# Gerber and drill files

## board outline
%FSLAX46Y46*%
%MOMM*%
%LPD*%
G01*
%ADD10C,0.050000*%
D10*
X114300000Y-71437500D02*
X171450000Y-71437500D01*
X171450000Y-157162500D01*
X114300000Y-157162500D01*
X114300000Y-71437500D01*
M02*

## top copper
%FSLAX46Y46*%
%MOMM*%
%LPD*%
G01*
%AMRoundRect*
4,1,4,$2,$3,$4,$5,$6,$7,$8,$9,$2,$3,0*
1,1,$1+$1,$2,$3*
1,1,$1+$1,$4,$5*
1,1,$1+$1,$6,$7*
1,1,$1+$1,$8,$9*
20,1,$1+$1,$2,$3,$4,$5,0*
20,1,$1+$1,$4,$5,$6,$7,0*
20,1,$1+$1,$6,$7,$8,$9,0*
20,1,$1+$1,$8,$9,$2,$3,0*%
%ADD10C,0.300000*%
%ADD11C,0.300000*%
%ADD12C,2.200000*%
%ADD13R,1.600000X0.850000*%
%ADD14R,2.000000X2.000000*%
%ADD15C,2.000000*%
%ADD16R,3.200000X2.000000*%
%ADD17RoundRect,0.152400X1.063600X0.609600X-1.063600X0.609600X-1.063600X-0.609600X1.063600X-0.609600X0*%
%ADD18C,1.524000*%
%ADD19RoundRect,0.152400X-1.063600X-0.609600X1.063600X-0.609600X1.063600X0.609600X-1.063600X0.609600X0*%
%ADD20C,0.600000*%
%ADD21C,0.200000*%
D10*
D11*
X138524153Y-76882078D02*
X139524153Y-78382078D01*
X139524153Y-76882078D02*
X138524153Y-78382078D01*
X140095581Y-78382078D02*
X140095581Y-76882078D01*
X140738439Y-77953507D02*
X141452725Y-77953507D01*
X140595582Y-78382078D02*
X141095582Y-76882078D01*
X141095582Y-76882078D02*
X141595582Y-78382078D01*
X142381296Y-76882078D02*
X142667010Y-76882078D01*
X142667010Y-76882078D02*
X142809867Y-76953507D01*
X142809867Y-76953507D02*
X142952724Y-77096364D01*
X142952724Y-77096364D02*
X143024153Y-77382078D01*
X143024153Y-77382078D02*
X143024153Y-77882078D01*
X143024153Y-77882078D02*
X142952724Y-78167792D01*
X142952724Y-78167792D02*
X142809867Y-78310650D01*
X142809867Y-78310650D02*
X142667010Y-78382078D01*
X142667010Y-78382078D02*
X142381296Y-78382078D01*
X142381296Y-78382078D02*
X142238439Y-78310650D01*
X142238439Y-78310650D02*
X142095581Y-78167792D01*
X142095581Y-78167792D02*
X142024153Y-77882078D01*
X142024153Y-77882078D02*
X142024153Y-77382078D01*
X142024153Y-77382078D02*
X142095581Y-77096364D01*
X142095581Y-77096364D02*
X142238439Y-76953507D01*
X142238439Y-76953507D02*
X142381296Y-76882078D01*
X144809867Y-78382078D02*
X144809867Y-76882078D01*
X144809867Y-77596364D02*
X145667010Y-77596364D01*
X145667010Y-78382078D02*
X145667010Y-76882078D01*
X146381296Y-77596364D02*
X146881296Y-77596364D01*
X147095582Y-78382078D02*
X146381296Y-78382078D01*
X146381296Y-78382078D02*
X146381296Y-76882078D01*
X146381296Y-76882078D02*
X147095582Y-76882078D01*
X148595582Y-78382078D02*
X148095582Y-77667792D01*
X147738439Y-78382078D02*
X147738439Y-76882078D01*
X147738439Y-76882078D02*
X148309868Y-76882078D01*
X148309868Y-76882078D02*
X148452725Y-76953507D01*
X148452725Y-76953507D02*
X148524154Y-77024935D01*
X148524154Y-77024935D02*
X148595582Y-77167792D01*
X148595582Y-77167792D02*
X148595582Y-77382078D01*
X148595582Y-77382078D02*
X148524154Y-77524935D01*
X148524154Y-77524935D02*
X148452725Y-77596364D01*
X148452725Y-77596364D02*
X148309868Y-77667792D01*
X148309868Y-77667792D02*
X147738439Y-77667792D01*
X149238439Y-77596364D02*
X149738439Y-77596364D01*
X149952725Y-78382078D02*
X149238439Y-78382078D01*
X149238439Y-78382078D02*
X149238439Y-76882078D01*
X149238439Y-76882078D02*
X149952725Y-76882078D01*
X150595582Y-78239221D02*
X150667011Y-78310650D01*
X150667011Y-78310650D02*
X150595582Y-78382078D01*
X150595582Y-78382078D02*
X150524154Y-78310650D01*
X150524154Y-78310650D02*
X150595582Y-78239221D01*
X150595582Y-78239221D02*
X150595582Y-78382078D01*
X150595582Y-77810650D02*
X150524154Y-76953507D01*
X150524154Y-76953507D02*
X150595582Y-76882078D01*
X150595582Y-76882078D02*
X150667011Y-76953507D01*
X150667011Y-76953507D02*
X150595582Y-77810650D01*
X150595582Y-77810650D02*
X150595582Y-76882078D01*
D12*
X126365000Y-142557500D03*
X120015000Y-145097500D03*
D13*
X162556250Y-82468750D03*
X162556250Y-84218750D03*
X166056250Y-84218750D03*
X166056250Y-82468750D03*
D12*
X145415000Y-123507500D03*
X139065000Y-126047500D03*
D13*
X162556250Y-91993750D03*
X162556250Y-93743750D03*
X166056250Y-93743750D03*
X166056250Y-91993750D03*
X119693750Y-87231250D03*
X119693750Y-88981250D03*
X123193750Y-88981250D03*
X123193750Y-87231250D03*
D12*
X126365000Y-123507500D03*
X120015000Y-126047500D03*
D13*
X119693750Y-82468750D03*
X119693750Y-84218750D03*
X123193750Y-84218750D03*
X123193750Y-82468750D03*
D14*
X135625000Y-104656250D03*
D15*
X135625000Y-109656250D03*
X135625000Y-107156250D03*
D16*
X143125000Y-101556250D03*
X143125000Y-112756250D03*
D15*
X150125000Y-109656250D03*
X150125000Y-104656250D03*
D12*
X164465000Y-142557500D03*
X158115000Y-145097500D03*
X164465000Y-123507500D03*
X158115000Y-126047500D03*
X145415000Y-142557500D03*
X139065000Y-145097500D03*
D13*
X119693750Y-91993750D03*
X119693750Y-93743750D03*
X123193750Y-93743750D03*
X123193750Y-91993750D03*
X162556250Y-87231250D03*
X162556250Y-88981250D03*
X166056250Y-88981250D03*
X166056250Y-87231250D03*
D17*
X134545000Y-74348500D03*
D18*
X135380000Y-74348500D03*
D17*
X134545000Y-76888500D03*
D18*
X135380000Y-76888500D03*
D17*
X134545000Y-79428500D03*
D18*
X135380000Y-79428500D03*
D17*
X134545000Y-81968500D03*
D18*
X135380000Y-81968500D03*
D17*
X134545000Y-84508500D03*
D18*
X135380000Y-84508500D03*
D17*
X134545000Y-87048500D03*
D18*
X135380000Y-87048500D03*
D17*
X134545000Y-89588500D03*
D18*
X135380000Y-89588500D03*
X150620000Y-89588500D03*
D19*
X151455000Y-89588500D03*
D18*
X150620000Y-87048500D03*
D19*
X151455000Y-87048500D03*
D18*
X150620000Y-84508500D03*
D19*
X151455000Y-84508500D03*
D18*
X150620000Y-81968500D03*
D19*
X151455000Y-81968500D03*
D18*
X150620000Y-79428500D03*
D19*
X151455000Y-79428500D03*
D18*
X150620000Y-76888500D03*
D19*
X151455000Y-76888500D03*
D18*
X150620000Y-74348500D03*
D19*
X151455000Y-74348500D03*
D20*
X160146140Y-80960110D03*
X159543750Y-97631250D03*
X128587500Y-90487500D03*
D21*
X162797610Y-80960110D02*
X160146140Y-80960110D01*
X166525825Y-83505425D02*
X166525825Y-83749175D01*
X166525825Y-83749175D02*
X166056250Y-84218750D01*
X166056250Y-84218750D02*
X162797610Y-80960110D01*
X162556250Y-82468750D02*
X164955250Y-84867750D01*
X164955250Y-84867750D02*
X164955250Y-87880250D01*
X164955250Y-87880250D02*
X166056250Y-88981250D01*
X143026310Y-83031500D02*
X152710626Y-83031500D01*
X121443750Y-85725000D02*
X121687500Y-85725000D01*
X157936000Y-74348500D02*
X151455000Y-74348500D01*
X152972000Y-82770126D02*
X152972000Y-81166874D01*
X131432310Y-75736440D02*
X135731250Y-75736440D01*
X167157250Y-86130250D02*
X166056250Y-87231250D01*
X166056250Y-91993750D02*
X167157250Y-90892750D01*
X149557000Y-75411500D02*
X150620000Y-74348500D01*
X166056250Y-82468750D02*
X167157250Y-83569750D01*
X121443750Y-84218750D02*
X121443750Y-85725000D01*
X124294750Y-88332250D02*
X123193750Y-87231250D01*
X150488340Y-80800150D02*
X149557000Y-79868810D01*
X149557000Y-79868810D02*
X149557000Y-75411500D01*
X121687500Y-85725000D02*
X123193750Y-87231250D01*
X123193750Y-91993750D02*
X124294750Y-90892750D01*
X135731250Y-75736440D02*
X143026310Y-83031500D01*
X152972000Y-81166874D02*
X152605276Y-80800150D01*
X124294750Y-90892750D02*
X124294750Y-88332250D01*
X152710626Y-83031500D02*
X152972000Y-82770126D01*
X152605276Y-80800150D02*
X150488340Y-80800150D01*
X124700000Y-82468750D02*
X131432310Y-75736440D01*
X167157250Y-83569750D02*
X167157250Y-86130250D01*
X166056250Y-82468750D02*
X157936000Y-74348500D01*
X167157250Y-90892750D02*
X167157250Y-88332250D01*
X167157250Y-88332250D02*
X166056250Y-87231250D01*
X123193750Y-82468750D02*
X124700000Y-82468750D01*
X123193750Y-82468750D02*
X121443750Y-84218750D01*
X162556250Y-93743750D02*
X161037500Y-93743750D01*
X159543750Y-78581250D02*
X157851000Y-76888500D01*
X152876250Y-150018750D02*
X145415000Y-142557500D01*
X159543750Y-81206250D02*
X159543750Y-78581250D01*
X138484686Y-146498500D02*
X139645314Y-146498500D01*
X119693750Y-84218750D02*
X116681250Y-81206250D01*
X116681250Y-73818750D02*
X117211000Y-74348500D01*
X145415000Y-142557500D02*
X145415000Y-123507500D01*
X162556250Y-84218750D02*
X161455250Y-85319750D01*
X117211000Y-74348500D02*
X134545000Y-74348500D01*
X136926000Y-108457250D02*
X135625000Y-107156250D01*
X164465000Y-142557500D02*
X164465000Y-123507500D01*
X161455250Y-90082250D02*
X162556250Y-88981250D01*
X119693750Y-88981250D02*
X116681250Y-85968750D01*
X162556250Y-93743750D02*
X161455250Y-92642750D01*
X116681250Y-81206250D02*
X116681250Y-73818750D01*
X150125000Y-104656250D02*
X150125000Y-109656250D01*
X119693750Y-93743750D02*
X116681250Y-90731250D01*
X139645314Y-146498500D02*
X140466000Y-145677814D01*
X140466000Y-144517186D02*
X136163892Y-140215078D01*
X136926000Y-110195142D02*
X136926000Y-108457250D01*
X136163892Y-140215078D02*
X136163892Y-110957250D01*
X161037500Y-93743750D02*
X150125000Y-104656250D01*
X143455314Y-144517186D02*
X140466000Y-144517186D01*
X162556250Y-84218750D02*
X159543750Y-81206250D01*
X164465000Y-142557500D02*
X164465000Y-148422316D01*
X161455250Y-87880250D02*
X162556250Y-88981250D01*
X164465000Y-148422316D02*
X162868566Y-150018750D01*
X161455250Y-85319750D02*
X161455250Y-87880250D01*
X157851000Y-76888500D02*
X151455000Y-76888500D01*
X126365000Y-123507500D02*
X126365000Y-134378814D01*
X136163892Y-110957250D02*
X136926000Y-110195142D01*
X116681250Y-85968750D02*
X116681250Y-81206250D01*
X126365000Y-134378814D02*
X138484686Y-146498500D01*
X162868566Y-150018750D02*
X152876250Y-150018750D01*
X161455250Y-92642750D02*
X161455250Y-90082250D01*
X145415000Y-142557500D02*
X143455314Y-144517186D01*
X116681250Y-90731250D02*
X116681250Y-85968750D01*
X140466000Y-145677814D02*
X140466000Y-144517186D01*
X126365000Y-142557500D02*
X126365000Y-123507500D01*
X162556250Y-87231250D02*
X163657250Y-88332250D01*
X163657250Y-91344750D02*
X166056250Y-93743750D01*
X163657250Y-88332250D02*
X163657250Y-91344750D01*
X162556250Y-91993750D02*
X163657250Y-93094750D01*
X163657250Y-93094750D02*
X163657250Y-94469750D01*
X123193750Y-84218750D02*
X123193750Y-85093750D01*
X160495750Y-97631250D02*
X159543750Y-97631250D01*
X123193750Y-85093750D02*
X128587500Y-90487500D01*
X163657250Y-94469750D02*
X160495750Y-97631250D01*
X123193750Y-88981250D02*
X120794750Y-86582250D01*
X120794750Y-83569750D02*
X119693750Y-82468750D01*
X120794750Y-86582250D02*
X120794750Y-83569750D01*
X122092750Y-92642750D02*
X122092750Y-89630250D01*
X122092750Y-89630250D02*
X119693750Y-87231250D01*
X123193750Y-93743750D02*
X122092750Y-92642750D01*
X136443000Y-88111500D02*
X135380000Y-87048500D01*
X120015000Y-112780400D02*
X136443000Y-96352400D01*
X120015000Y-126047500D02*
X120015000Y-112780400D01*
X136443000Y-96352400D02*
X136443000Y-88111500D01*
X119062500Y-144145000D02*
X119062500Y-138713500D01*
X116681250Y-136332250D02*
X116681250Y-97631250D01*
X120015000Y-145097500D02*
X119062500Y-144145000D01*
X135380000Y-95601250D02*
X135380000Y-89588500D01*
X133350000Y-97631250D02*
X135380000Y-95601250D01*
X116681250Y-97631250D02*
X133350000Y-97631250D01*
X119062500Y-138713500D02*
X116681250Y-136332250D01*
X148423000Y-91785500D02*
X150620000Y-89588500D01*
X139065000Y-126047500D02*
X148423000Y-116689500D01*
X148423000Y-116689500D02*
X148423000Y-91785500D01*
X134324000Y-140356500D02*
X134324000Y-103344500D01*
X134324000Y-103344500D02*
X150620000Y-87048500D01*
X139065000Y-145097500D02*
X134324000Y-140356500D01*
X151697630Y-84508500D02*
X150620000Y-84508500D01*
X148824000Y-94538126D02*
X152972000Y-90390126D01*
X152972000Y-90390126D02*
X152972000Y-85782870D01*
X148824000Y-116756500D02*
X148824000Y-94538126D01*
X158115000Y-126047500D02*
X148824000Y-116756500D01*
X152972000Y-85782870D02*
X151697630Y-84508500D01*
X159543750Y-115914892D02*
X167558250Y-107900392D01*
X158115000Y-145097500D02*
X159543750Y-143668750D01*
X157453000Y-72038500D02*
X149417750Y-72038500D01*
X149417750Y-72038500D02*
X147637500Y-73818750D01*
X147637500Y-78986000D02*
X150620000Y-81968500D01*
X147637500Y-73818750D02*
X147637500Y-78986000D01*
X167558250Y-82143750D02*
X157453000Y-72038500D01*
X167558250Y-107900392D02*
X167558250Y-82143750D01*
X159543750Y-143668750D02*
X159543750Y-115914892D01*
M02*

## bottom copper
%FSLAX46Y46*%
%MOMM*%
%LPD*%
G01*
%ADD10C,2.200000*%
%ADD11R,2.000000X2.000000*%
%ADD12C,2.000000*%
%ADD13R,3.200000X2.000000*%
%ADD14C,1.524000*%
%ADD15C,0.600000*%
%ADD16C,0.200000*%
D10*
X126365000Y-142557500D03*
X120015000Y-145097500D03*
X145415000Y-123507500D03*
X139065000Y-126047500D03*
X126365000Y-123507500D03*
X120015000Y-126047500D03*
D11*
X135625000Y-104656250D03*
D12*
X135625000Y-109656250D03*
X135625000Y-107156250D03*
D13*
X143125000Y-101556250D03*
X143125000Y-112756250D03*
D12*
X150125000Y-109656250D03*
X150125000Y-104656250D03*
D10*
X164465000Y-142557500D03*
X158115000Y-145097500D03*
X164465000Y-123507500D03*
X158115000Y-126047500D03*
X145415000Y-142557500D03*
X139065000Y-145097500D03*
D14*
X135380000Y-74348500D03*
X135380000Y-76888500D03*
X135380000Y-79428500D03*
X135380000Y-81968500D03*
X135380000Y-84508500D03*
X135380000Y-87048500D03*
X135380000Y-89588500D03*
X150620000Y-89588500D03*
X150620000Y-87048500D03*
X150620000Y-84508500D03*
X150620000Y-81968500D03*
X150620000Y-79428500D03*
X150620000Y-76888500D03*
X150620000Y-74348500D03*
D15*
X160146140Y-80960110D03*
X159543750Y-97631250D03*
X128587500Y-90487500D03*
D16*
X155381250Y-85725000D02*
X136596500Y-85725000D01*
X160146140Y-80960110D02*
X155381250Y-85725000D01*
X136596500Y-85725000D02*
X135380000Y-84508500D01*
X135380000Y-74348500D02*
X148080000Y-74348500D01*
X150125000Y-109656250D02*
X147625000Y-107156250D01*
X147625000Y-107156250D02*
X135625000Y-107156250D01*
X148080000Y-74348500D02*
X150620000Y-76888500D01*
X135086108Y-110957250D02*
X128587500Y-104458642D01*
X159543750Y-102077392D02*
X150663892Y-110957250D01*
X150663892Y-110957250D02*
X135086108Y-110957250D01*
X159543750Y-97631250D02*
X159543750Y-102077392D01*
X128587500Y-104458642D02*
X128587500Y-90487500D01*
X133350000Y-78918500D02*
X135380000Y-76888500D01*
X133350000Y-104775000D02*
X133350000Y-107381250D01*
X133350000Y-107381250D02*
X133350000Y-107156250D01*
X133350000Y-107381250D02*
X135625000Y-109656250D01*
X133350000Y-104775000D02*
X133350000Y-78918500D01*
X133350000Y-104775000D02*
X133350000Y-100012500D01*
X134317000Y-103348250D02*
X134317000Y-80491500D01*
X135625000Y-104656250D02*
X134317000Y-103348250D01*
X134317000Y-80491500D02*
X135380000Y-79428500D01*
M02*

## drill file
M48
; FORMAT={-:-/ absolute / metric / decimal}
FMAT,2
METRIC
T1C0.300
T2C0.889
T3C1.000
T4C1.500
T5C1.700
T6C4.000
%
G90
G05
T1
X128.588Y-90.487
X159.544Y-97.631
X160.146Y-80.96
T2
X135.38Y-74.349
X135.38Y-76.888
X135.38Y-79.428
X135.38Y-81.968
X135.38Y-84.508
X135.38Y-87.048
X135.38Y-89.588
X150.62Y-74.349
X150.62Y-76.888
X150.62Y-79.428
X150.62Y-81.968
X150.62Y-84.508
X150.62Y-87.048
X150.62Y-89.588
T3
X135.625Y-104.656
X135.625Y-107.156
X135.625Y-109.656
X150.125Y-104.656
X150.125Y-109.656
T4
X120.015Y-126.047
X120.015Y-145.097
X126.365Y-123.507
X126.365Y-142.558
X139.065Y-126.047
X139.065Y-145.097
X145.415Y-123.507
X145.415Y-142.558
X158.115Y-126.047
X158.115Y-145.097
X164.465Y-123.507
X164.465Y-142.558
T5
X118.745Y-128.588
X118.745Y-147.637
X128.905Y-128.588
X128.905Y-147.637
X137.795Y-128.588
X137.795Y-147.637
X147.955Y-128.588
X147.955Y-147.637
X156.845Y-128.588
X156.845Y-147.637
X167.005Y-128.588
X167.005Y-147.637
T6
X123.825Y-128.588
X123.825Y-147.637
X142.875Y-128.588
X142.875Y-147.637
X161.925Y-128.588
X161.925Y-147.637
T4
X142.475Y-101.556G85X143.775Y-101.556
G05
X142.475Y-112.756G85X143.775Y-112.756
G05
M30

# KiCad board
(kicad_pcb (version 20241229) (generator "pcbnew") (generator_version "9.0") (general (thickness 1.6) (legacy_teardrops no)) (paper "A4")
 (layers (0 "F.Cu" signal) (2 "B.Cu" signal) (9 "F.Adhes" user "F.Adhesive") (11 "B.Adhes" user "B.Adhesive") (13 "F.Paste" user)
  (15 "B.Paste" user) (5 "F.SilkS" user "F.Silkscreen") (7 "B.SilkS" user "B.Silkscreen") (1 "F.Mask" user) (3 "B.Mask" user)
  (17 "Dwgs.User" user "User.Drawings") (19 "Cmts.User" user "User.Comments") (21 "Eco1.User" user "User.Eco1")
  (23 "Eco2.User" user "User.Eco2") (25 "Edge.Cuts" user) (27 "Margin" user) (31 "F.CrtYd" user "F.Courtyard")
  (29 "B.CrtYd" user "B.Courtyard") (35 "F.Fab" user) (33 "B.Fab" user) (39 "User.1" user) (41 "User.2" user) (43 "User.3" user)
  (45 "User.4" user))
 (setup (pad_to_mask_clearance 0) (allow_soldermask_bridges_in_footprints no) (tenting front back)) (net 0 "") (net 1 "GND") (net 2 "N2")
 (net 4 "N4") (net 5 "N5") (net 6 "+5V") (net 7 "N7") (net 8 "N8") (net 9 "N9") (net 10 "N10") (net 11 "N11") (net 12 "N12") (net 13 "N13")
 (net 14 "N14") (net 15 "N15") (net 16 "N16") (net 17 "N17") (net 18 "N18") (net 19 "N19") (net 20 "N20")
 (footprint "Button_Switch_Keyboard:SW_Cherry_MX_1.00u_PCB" (layer "F.Cu") (at 126.365 142.5575)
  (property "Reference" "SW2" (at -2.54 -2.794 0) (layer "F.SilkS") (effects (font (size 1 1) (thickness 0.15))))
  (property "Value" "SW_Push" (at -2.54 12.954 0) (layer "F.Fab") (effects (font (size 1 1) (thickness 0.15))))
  (pad "" np_thru_hole circle (at -7.62 5.08) (size 1.7 1.7) (drill 1.7) (layers "*.Cu" "*.Mask"))
  (pad "" np_thru_hole circle (at -2.54 5.08) (size 4 4) (drill 4) (layers "*.Cu" "*.Mask"))
  (pad "" np_thru_hole circle (at 2.54 5.08) (size 1.7 1.7) (drill 1.7) (layers "*.Cu" "*.Mask"))
  (pad "1" thru_hole circle (at 0 0) (size 2.2 2.2) (drill 1.5) (layers "*.Cu" "*.Mask") (remove_unused_layers no) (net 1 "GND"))
  (pad "2" thru_hole circle (at -6.35 2.54) (size 2.2 2.2) (drill 1.5) (layers "*.Cu" "*.Mask") (remove_unused_layers no) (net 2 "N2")))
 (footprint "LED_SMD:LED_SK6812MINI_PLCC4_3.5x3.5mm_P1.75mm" (layer "F.Cu") (at 164.30625 83.34375)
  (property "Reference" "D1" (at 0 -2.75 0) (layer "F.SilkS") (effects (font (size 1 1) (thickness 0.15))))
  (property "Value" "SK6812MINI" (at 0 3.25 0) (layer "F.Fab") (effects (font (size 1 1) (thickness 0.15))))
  (pad "1" smd rect (at -1.75 -0.875) (size 1.6 0.85) (layers "F.Cu" "F.Mask" "F.Paste") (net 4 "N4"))
  (pad "2" smd rect (at -1.75 0.875) (size 1.6 0.85) (layers "F.Cu" "F.Mask" "F.Paste") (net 1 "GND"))
  (pad "3" smd rect (at 1.75 0.875) (size 1.6 0.85) (layers "F.Cu" "F.Mask" "F.Paste") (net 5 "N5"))
  (pad "4" smd rect (at 1.75 -0.875) (size 1.6 0.85) (layers "F.Cu" "F.Mask" "F.Paste") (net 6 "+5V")))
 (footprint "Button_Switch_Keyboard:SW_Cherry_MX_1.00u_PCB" (layer "F.Cu") (at 145.415 123.5075)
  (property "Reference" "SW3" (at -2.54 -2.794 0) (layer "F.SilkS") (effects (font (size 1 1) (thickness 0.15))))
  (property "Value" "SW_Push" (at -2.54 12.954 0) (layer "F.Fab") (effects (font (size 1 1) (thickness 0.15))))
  (pad "" np_thru_hole circle (at -7.62 5.08) (size 1.7 1.7) (drill 1.7) (layers "*.Cu" "*.Mask"))
  (pad "" np_thru_hole circle (at -2.54 5.08) (size 4 4) (drill 4) (layers "*.Cu" "*.Mask"))
  (pad "" np_thru_hole circle (at 2.54 5.08) (size 1.7 1.7) (drill 1.7) (layers "*.Cu" "*.Mask"))
  (pad "1" thru_hole circle (at 0 0) (size 2.2 2.2) (drill 1.5) (layers "*.Cu" "*.Mask") (remove_unused_layers no) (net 1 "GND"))
  (pad "2" thru_hole circle (at -6.35 2.54) (size 2.2 2.2) (drill 1.5) (layers "*.Cu" "*.Mask") (remove_unused_layers no) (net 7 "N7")))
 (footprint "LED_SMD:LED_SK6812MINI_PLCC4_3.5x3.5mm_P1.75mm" (layer "F.Cu") (at 164.30625 92.86875)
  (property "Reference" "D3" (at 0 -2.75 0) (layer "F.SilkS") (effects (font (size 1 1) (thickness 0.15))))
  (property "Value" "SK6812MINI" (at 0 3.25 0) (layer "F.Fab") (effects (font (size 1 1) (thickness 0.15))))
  (pad "1" smd rect (at -1.75 -0.875) (size 1.6 0.85) (layers "F.Cu" "F.Mask" "F.Paste") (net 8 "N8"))
  (pad "2" smd rect (at -1.75 0.875) (size 1.6 0.85) (layers "F.Cu" "F.Mask" "F.Paste") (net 1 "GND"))
  (pad "3" smd rect (at 1.75 0.875) (size 1.6 0.85) (layers "F.Cu" "F.Mask" "F.Paste") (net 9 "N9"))
  (pad "4" smd rect (at 1.75 -0.875) (size 1.6 0.85) (layers "F.Cu" "F.Mask" "F.Paste") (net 6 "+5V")))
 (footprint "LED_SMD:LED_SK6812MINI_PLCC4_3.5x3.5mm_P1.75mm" (layer "F.Cu") (at 121.44375 88.10625)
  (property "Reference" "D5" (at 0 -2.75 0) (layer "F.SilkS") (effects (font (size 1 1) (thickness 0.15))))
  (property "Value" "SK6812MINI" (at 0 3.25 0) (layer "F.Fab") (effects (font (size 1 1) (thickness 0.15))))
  (pad "1" smd rect (at -1.75 -0.875) (size 1.6 0.85) (layers "F.Cu" "F.Mask" "F.Paste") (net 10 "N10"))
  (pad "2" smd rect (at -1.75 0.875) (size 1.6 0.85) (layers "F.Cu" "F.Mask" "F.Paste") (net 1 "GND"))
  (pad "3" smd rect (at 1.75 0.875) (size 1.6 0.85) (layers "F.Cu" "F.Mask" "F.Paste") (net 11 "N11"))
  (pad "4" smd rect (at 1.75 -0.875) (size 1.6 0.85) (layers "F.Cu" "F.Mask" "F.Paste") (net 6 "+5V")))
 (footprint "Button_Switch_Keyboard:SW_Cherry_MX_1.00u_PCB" (layer "F.Cu") (at 126.365 123.5075)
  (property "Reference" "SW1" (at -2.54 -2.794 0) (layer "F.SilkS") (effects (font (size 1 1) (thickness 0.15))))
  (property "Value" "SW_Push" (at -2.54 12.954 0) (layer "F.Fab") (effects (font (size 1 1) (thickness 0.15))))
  (pad "" np_thru_hole circle (at -7.62 5.08) (size 1.7 1.7) (drill 1.7) (layers "*.Cu" "*.Mask"))
  (pad "" np_thru_hole circle (at -2.54 5.08) (size 4 4) (drill 4) (layers "*.Cu" "*.Mask"))
  (pad "" np_thru_hole circle (at 2.54 5.08) (size 1.7 1.7) (drill 1.7) (layers "*.Cu" "*.Mask"))
  (pad "1" thru_hole circle (at 0 0) (size 2.2 2.2) (drill 1.5) (layers "*.Cu" "*.Mask") (remove_unused_layers no) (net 1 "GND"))
  (pad "2" thru_hole circle (at -6.35 2.54) (size 2.2 2.2) (drill 1.5) (layers "*.Cu" "*.Mask") (remove_unused_layers no) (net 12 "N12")))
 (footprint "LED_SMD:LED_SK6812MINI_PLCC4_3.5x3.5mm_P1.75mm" (layer "F.Cu") (at 121.44375 83.34375)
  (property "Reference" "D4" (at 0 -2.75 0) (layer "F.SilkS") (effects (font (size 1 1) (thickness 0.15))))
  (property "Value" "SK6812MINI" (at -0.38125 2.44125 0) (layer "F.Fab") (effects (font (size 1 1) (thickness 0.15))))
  (pad "1" smd rect (at -1.75 -0.875) (size 1.6 0.85) (layers "F.Cu" "F.Mask" "F.Paste") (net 11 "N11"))
  (pad "2" smd rect (at -1.75 0.875) (size 1.6 0.85) (layers "F.Cu" "F.Mask" "F.Paste") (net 1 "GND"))
  (pad "3" smd rect (at 1.75 0.875) (size 1.6 0.85) (layers "F.Cu" "F.Mask" "F.Paste") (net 8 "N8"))
  (pad "4" smd rect (at 1.75 -0.875) (size 1.6 0.85) (layers "F.Cu" "F.Mask" "F.Paste") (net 6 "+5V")))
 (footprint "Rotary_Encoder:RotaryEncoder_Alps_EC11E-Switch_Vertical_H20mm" (layer "F.Cu") (at 135.625 104.65625)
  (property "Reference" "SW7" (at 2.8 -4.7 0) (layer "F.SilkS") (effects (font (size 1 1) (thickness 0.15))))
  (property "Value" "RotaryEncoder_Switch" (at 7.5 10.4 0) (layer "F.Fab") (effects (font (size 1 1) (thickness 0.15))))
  (pad "A" thru_hole rect (at 0 0) (size 2 2) (drill 1) (layers "*.Cu" "*.Mask") (remove_unused_layers no) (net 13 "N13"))
  (pad "B" thru_hole circle (at 0 5) (size 2 2) (drill 1) (layers "*.Cu" "*.Mask") (remove_unused_layers no) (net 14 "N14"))
  (pad "C" thru_hole circle (at 0 2.5) (size 2 2) (drill 1) (layers "*.Cu" "*.Mask") (remove_unused_layers no) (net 1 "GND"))
  (pad "MP" thru_hole rect (at 7.5 -3.1) (size 3.2 2) (drill oval 2.8 1.5) (layers "*.Cu" "*.Mask") (remove_unused_layers no))
  (pad "MP" thru_hole rect (at 7.5 8.1) (size 3.2 2) (drill oval 2.8 1.5) (layers "*.Cu" "*.Mask") (remove_unused_layers no))
  (pad "S1" thru_hole circle (at 14.5 5) (size 2 2) (drill 1) (layers "*.Cu" "*.Mask") (remove_unused_layers no) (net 1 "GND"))
  (pad "S2" thru_hole circle (at 14.5 0) (size 2 2) (drill 1) (layers "*.Cu" "*.Mask") (remove_unused_layers no) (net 1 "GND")))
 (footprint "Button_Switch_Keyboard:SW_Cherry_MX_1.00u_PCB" (layer "F.Cu") (at 164.465 142.5575)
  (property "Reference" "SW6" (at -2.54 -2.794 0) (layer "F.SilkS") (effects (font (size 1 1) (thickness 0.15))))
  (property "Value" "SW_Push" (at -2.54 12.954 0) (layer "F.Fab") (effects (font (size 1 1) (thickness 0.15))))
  (pad "" np_thru_hole circle (at -7.62 5.08) (size 1.7 1.7) (drill 1.7) (layers "*.Cu" "*.Mask"))
  (pad "" np_thru_hole circle (at -2.54 5.08) (size 4 4) (drill 4) (layers "*.Cu" "*.Mask"))
  (pad "" np_thru_hole circle (at 2.54 5.08) (size 1.7 1.7) (drill 1.7) (layers "*.Cu" "*.Mask"))
  (pad "1" thru_hole circle (at 0 0) (size 2.2 2.2) (drill 1.5) (layers "*.Cu" "*.Mask") (remove_unused_layers no) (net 1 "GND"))
  (pad "2" thru_hole circle (at -6.35 2.54) (size 2.2 2.2) (drill 1.5) (layers "*.Cu" "*.Mask") (remove_unused_layers no) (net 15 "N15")))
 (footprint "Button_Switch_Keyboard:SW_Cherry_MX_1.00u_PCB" (layer "F.Cu") (at 164.465 123.5075)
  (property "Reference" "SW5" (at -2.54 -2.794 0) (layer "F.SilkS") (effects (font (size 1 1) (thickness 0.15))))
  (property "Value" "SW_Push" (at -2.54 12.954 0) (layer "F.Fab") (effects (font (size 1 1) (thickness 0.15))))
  (pad "" np_thru_hole circle (at -7.62 5.08) (size 1.7 1.7) (drill 1.7) (layers "*.Cu" "*.Mask"))
  (pad "" np_thru_hole circle (at -2.54 5.08) (size 4 4) (drill 4) (layers "*.Cu" "*.Mask"))
  (pad "" np_thru_hole circle (at 2.54 5.08) (size 1.7 1.7) (drill 1.7) (layers "*.Cu" "*.Mask"))
  (pad "1" thru_hole circle (at 0 0) (size 2.2 2.2) (drill 1.5) (layers "*.Cu" "*.Mask") (remove_unused_layers no) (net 1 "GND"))
  (pad "2" thru_hole circle (at -6.35 2.54) (size 2.2 2.2) (drill 1.5) (layers "*.Cu" "*.Mask") (remove_unused_layers no) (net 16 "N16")))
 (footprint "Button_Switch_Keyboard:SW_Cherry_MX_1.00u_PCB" (layer "F.Cu") (at 145.415 142.5575)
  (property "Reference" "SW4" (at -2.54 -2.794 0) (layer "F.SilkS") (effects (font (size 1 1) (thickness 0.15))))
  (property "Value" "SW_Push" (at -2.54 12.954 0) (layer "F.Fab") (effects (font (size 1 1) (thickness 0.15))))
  (pad "" np_thru_hole circle (at -7.62 5.08) (size 1.7 1.7) (drill 1.7) (layers "*.Cu" "*.Mask"))
  (pad "" np_thru_hole circle (at -2.54 5.08) (size 4 4) (drill 4) (layers "*.Cu" "*.Mask"))
  (pad "" np_thru_hole circle (at 2.54 5.08) (size 1.7 1.7) (drill 1.7) (layers "*.Cu" "*.Mask"))
  (pad "1" thru_hole circle (at 0 0) (size 2.2 2.2) (drill 1.5) (layers "*.Cu" "*.Mask") (remove_unused_layers no) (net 1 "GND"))
  (pad "2" thru_hole circle (at -6.35 2.54) (size 2.2 2.2) (drill 1.5) (layers "*.Cu" "*.Mask") (remove_unused_layers no) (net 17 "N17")))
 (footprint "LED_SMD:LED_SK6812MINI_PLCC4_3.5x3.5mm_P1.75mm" (layer "F.Cu") (at 121.44375 92.86875)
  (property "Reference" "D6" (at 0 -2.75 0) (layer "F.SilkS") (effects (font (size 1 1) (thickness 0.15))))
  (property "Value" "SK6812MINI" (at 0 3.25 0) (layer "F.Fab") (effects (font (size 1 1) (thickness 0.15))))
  (pad "1" smd rect (at -1.75 -0.875) (size 1.6 0.85) (layers "F.Cu" "F.Mask" "F.Paste") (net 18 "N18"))
  (pad "2" smd rect (at -1.75 0.875) (size 1.6 0.85) (layers "F.Cu" "F.Mask" "F.Paste") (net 1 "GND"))
  (pad "3" smd rect (at 1.75 0.875) (size 1.6 0.85) (layers "F.Cu" "F.Mask" "F.Paste") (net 10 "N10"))
  (pad "4" smd rect (at 1.75 -0.875) (size 1.6 0.85) (layers "F.Cu" "F.Mask" "F.Paste") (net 6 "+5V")))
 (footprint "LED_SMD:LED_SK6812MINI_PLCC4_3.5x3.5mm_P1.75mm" (layer "F.Cu") (at 164.30625 88.10625)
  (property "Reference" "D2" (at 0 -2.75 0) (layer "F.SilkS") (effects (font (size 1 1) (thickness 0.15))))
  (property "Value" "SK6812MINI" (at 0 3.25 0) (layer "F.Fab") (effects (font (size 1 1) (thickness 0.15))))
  (pad "1" smd rect (at -1.75 -0.875) (size 1.6 0.85) (layers "F.Cu" "F.Mask" "F.Paste") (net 9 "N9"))
  (pad "2" smd rect (at -1.75 0.875) (size 1.6 0.85) (layers "F.Cu" "F.Mask" "F.Paste") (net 1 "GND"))
  (pad "3" smd rect (at 1.75 0.875) (size 1.6 0.85) (layers "F.Cu" "F.Mask" "F.Paste") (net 4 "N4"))
  (pad "4" smd rect (at 1.75 -0.875) (size 1.6 0.85) (layers "F.Cu" "F.Mask" "F.Paste") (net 6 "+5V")))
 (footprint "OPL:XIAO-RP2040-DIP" (layer "F.Cu") (at 143 81.9685)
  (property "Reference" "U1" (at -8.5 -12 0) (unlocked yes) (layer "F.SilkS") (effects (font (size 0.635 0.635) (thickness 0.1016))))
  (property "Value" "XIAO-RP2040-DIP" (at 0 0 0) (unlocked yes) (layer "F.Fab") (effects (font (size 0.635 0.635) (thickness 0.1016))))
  (pad "1" smd roundrect (at -8.455 -7.62 180) (size 2.432 1.524) (layers "F.Cu" "F.Mask") (roundrect_rratio 0.1) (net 1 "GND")
   (thermal_bridge_angle 45))
  (pad "1" thru_hole circle (at -7.62 -7.62 180) (size 1.524 1.524) (drill 0.889) (layers "*.Cu" "*.Mask") (remove_unused_layers no)
   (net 1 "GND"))
  (pad "2" smd roundrect (at -8.455 -5.08 180) (size 2.432 1.524) (layers "F.Cu" "F.Mask") (roundrect_rratio 0.1) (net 14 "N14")
   (thermal_bridge_angle 45))
  (pad "2" thru_hole circle (at -7.62 -5.08 180) (size 1.524 1.524) (drill 0.889) (layers "*.Cu" "*.Mask") (remove_unused_layers no)
   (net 14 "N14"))
  (pad "3" smd roundrect (at -8.455 -2.54 180) (size 2.432 1.524) (layers "F.Cu" "F.Mask") (roundrect_rratio 0.1) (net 13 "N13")
   (thermal_bridge_angle 45))
  (pad "3" thru_hole circle (at -7.62 -2.54 180) (size 1.524 1.524) (drill 0.889) (layers "*.Cu" "*.Mask") (remove_unused_layers no)
   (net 13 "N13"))
  (pad "4" smd roundrect (at -8.455 0 180) (size 2.432 1.524) (layers "F.Cu" "F.Mask") (roundrect_rratio 0.1) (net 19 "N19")
   (thermal_bridge_angle 45))
  (pad "4" thru_hole circle (at -7.62 0 180) (size 1.524 1.524) (drill 0.889) (layers "*.Cu" "*.Mask") (remove_unused_layers no)
   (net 19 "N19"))
  (pad "5" smd roundrect (at -8.455 2.54 180) (size 2.432 1.524) (layers "F.Cu" "F.Mask") (roundrect_rratio 0.1) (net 5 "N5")
   (thermal_bridge_angle 45))
  (pad "5" thru_hole circle (at -7.62 2.54 180) (size 1.524 1.524) (drill 0.889) (layers "*.Cu" "*.Mask") (remove_unused_layers no)
   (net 5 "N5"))
  (pad "6" smd roundrect (at -8.455 5.08 180) (size 2.432 1.524) (layers "F.Cu" "F.Mask") (roundrect_rratio 0.1) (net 12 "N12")
   (thermal_bridge_angle 45))
  (pad "6" thru_hole circle (at -7.62 5.08 180) (size 1.524 1.524) (drill 0.889) (layers "*.Cu" "*.Mask") (remove_unused_layers no)
   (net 12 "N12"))
  (pad "7" smd roundrect (at -8.455 7.62 180) (size 2.432 1.524) (layers "F.Cu" "F.Mask") (roundrect_rratio 0.1) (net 2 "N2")
   (thermal_bridge_angle 45))
  (pad "7" thru_hole circle (at -7.62 7.62 180) (size 1.524 1.524) (drill 0.889) (layers "*.Cu" "*.Mask") (remove_unused_layers no)
   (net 2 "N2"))
  (pad "8" thru_hole circle (at 7.62 7.62) (size 1.524 1.524) (drill 0.889) (layers "*.Cu" "*.Mask") (remove_unused_layers no) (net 7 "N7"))
  (pad "8" smd roundrect (at 8.455 7.62) (size 2.432 1.524) (layers "F.Cu" "F.Mask") (roundrect_rratio 0.1) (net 7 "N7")
   (thermal_bridge_angle 45))
  (pad "9" thru_hole circle (at 7.62 5.08) (size 1.524 1.524) (drill 0.889) (layers "*.Cu" "*.Mask") (remove_unused_layers no)
   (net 17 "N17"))
  (pad "9" smd roundrect (at 8.455 5.08) (size 2.432 1.524) (layers "F.Cu" "F.Mask") (roundrect_rratio 0.1) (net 17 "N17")
   (thermal_bridge_angle 45))
  (pad "10" thru_hole circle (at 7.62 2.54) (size 1.524 1.524) (drill 0.889) (layers "*.Cu" "*.Mask") (remove_unused_layers no)
   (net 16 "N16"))
  (pad "10" smd roundrect (at 8.455 2.54) (size 2.432 1.524) (layers "F.Cu" "F.Mask") (roundrect_rratio 0.1) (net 16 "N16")
   (thermal_bridge_angle 45))
  (pad "11" thru_hole circle (at 7.62 0) (size 1.524 1.524) (drill 0.889) (layers "*.Cu" "*.Mask") (remove_unused_layers no) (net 15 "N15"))
  (pad "11" smd roundrect (at 8.455 0) (size 2.432 1.524) (layers "F.Cu" "F.Mask") (roundrect_rratio 0.1) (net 15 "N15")
   (thermal_bridge_angle 45))
  (pad "12" thru_hole circle (at 7.62 -2.54) (size 1.524 1.524) (drill 0.889) (layers "*.Cu" "*.Mask") (remove_unused_layers no)
   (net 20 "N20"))
  (pad "12" smd roundrect (at 8.455 -2.54) (size 2.432 1.524) (layers "F.Cu" "F.Mask") (roundrect_rratio 0.1) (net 20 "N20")
   (thermal_bridge_angle 45))
  (pad "13" thru_hole circle (at 7.62 -5.08) (size 1.524 1.524) (drill 0.889) (layers "*.Cu" "*.Mask") (remove_unused_layers no)
   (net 1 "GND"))
  (pad "13" smd roundrect (at 8.455 -5.08) (size 2.432 1.524) (layers "F.Cu" "F.Mask") (roundrect_rratio 0.1) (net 1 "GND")
   (thermal_bridge_angle 45))
  (pad "14" thru_hole circle (at 7.62 -7.62) (size 1.524 1.524) (drill 0.889) (layers "*.Cu" "*.Mask") (remove_unused_layers no)
   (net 6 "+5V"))
  (pad "14" smd roundrect (at 8.455 -7.62) (size 2.432 1.524) (layers "F.Cu" "F.Mask") (roundrect_rratio 0.1) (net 6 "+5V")
   (thermal_bridge_angle 45)))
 (gr_rect (start 114.3 71.4375) (end 171.45 157.1625) (stroke (width 0.05) (type default)) (fill no) (layer "Edge.Cuts"))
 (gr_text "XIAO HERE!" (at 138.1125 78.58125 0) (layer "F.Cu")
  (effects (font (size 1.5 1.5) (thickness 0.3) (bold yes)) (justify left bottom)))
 (segment (start 162.79761 80.96011) (end 160.14614 80.96011) (width 0.2) (layer "F.Cu") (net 5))
 (segment (start 166.525825 83.505425) (end 166.525825 83.749175) (width 0.2) (layer "F.Cu") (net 5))
 (segment (start 166.525825 83.749175) (end 166.05625 84.21875) (width 0.2) (layer "F.Cu") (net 5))
 (segment (start 166.05625 84.21875) (end 162.79761 80.96011) (width 0.2) (layer "F.Cu") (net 5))
 (via (at 160.14614 80.96011) (size 0.6) (drill 0.3) (layers "F.Cu" "B.Cu") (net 5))
 (segment (start 155.38125 85.725) (end 136.5965 85.725) (width 0.2) (layer "B.Cu") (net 5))
 (segment (start 160.14614 80.96011) (end 155.38125 85.725) (width 0.2) (layer "B.Cu") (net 5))
 (segment (start 136.5965 85.725) (end 135.38 84.5085) (width 0.2) (layer "B.Cu") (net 5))
 (segment (start 162.55625 82.46875) (end 164.95525 84.86775) (width 0.2) (layer "F.Cu") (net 4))
 (segment (start 164.95525 84.86775) (end 164.95525 87.88025) (width 0.2) (layer "F.Cu") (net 4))
 (segment (start 164.95525 87.88025) (end 166.05625 88.98125) (width 0.2) (layer "F.Cu") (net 4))
 (segment (start 143.02631 83.0315) (end 152.710626 83.0315) (width 0.2) (layer "F.Cu") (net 6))
 (segment (start 121.44375 85.725) (end 121.6875 85.725) (width 0.2) (layer "F.Cu") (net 6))
 (segment (start 157.936 74.3485) (end 151.455 74.3485) (width 0.2) (layer "F.Cu") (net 6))
 (segment (start 152.972 82.770126) (end 152.972 81.166874) (width 0.2) (layer "F.Cu") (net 6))
 (segment (start 131.43231 75.73644) (end 135.73125 75.73644) (width 0.2) (layer "F.Cu") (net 6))
 (segment (start 167.15725 86.13025) (end 166.05625 87.23125) (width 0.2) (layer "F.Cu") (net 6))
 (segment (start 166.05625 91.99375) (end 167.15725 90.89275) (width 0.2) (layer "F.Cu") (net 6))
 (segment (start 149.557 75.4115) (end 150.62 74.3485) (width 0.2) (layer "F.Cu") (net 6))
 (segment (start 166.05625 82.46875) (end 167.15725 83.56975) (width 0.2) (layer "F.Cu") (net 6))
 (segment (start 121.44375 84.21875) (end 121.44375 85.725) (width 0.2) (layer "F.Cu") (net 6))
 (segment (start 124.29475 88.33225) (end 123.19375 87.23125) (width 0.2) (layer "F.Cu") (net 6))
 (segment (start 150.48834 80.80015) (end 149.557 79.86881) (width 0.2) (layer "F.Cu") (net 6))
 (segment (start 149.557 79.86881) (end 149.557 75.4115) (width 0.2) (layer "F.Cu") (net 6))
 (segment (start 121.6875 85.725) (end 123.19375 87.23125) (width 0.2) (layer "F.Cu") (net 6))
 (segment (start 123.19375 91.99375) (end 124.29475 90.89275) (width 0.2) (layer "F.Cu") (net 6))
 (segment (start 135.73125 75.73644) (end 143.02631 83.0315) (width 0.2) (layer "F.Cu") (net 6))
 (segment (start 152.972 81.166874) (end 152.605276 80.80015) (width 0.2) (layer "F.Cu") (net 6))
 (segment (start 124.29475 90.89275) (end 124.29475 88.33225) (width 0.2) (layer "F.Cu") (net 6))
 (segment (start 152.710626 83.0315) (end 152.972 82.770126) (width 0.2) (layer "F.Cu") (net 6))
 (segment (start 152.605276 80.80015) (end 150.48834 80.80015) (width 0.2) (layer "F.Cu") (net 6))
 (segment (start 124.7 82.46875) (end 131.43231 75.73644) (width 0.2) (layer "F.Cu") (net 6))
 (segment (start 167.15725 83.56975) (end 167.15725 86.13025) (width 0.2) (layer "F.Cu") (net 6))
 (segment (start 166.05625 82.46875) (end 157.936 74.3485) (width 0.2) (layer "F.Cu") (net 6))
 (segment (start 167.15725 90.89275) (end 167.15725 88.33225) (width 0.2) (layer "F.Cu") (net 6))
 (segment (start 167.15725 88.33225) (end 166.05625 87.23125) (width 0.2) (layer "F.Cu") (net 6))
 (segment (start 123.19375 82.46875) (end 124.7 82.46875) (width 0.2) (layer "F.Cu") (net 6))
 (segment (start 123.19375 82.46875) (end 121.44375 84.21875) (width 0.2) (layer "F.Cu") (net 6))
 (segment (start 162.55625 93.74375) (end 161.0375 93.74375) (width 0.2) (layer "F.Cu") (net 1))
 (segment (start 159.54375 78.58125) (end 157.851 76.8885) (width 0.2) (layer "F.Cu") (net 1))
 (segment (start 152.87625 150.01875) (end 145.415 142.5575) (width 0.2) (layer "F.Cu") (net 1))
 (segment (start 159.54375 81.20625) (end 159.54375 78.58125) (width 0.2) (layer "F.Cu") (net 1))
 (segment (start 138.484686 146.4985) (end 139.645314 146.4985) (width 0.2) (layer "F.Cu") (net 1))
 (segment (start 119.69375 84.21875) (end 116.68125 81.20625) (width 0.2) (layer "F.Cu") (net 1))
 (segment (start 116.68125 73.81875) (end 117.211 74.3485) (width 0.2) (layer "F.Cu") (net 1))
 (segment (start 145.415 142.5575) (end 145.415 123.5075) (width 0.2) (layer "F.Cu") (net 1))
 (segment (start 162.55625 84.21875) (end 161.45525 85.31975) (width 0.2) (layer "F.Cu") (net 1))
 (segment (start 117.211 74.3485) (end 134.545 74.3485) (width 0.2) (layer "F.Cu") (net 1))
 (segment (start 136.926 108.45725) (end 135.625 107.15625) (width 0.2) (layer "F.Cu") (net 1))
 (segment (start 164.465 142.5575) (end 164.465 123.5075) (width 0.2) (layer "F.Cu") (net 1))
 (segment (start 161.45525 90.08225) (end 162.55625 88.98125) (width 0.2) (layer "F.Cu") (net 1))
 (segment (start 119.69375 88.98125) (end 116.68125 85.96875) (width 0.2) (layer "F.Cu") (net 1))
 (segment (start 162.55625 93.74375) (end 161.45525 92.64275) (width 0.2) (layer "F.Cu") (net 1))
 (segment (start 116.68125 81.20625) (end 116.68125 73.81875) (width 0.2) (layer "F.Cu") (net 1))
 (segment (start 150.125 104.65625) (end 150.125 109.65625) (width 0.2) (layer "F.Cu") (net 1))
 (segment (start 119.69375 93.74375) (end 116.68125 90.73125) (width 0.2) (layer "F.Cu") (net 1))
 (segment (start 139.645314 146.4985) (end 140.466 145.677814) (width 0.2) (layer "F.Cu") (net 1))
 (segment (start 140.466 144.517186) (end 136.163892 140.215078) (width 0.2) (layer "F.Cu") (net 1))
 (segment (start 136.926 110.195142) (end 136.926 108.45725) (width 0.2) (layer "F.Cu") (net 1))
 (segment (start 136.163892 140.215078) (end 136.163892 110.95725) (width 0.2) (layer "F.Cu") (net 1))
 (segment (start 161.0375 93.74375) (end 150.125 104.65625) (width 0.2) (layer "F.Cu") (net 1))
 (segment (start 143.455314 144.517186) (end 140.466 144.517186) (width 0.2) (layer "F.Cu") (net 1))
 (segment (start 162.55625 84.21875) (end 159.54375 81.20625) (width 0.2) (layer "F.Cu") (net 1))
 (segment (start 164.465 142.5575) (end 164.465 148.422316) (width 0.2) (layer "F.Cu") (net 1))
 (segment (start 161.45525 87.88025) (end 162.55625 88.98125) (width 0.2) (layer "F.Cu") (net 1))
 (segment (start 164.465 148.422316) (end 162.868566 150.01875) (width 0.2) (layer "F.Cu") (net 1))
 (segment (start 161.45525 85.31975) (end 161.45525 87.88025) (width 0.2) (layer "F.Cu") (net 1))
 (segment (start 157.851 76.8885) (end 151.455 76.8885) (width 0.2) (layer "F.Cu") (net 1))
 (segment (start 126.365 123.5075) (end 126.365 134.378814) (width 0.2) (layer "F.Cu") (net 1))
 (segment (start 136.163892 110.95725) (end 136.926 110.195142) (width 0.2) (layer "F.Cu") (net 1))
 (segment (start 116.68125 85.96875) (end 116.68125 81.20625) (width 0.2) (layer "F.Cu") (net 1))
 (segment (start 126.365 134.378814) (end 138.484686 146.4985) (width 0.2) (layer "F.Cu") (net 1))
 (segment (start 162.868566 150.01875) (end 152.87625 150.01875) (width 0.2) (layer "F.Cu") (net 1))
 (segment (start 161.45525 92.64275) (end 161.45525 90.08225) (width 0.2) (layer "F.Cu") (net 1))
 (segment (start 145.415 142.5575) (end 143.455314 144.517186) (width 0.2) (layer "F.Cu") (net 1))
 (segment (start 116.68125 90.73125) (end 116.68125 85.96875) (width 0.2) (layer "F.Cu") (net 1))
 (segment (start 140.466 145.677814) (end 140.466 144.517186) (width 0.2) (layer "F.Cu") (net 1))
 (segment (start 126.365 142.5575) (end 126.365 123.5075) (width 0.2) (layer "F.Cu") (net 1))
 (segment (start 135.38 74.3485) (end 148.08 74.3485) (width 0.2) (layer "B.Cu") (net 1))
 (segment (start 150.125 109.65625) (end 147.625 107.15625) (width 0.2) (layer "B.Cu") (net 1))
 (segment (start 147.625 107.15625) (end 135.625 107.15625) (width 0.2) (layer "B.Cu") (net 1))
 (segment (start 148.08 74.3485) (end 150.62 76.8885) (width 0.2) (layer "B.Cu") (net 1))
 (segment (start 162.55625 87.23125) (end 163.65725 88.33225) (width 0.2) (layer "F.Cu") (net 9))
 (segment (start 163.65725 91.34475) (end 166.05625 93.74375) (width 0.2) (layer "F.Cu") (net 9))
 (segment (start 163.65725 88.33225) (end 163.65725 91.34475) (width 0.2) (layer "F.Cu") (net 9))
 (segment (start 162.55625 91.99375) (end 163.65725 93.09475) (width 0.2) (layer "F.Cu") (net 8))
 (segment (start 163.65725 93.09475) (end 163.65725 94.46975) (width 0.2) (layer "F.Cu") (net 8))
 (segment (start 123.19375 84.21875) (end 123.19375 85.09375) (width 0.2) (layer "F.Cu") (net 8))
 (segment (start 160.49575 97.63125) (end 159.54375 97.63125) (width 0.2) (layer "F.Cu") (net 8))
 (segment (start 123.19375 85.09375) (end 128.5875 90.4875) (width 0.2) (layer "F.Cu") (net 8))
 (segment (start 163.65725 94.46975) (end 160.49575 97.63125) (width 0.2) (layer "F.Cu") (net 8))
 (via (at 159.54375 97.63125) (size 0.6) (drill 0.3) (layers "F.Cu" "B.Cu") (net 8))
 (via (at 128.5875 90.4875) (size 0.6) (drill 0.3) (layers "F.Cu" "B.Cu") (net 8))
 (segment (start 135.086108 110.95725) (end 128.5875 104.458642) (width 0.2) (layer "B.Cu") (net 8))
 (segment (start 159.54375 102.077392) (end 150.663892 110.95725) (width 0.2) (layer "B.Cu") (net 8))
 (segment (start 150.663892 110.95725) (end 135.086108 110.95725) (width 0.2) (layer "B.Cu") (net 8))
 (segment (start 159.54375 97.63125) (end 159.54375 102.077392) (width 0.2) (layer "B.Cu") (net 8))
 (segment (start 128.5875 104.458642) (end 128.5875 90.4875) (width 0.2) (layer "B.Cu") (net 8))
 (segment (start 123.19375 88.98125) (end 120.79475 86.58225) (width 0.2) (layer "F.Cu") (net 11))
 (segment (start 120.79475 83.56975) (end 119.69375 82.46875) (width 0.2) (layer "F.Cu") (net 11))
 (segment (start 120.79475 86.58225) (end 120.79475 83.56975) (width 0.2) (layer "F.Cu") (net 11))
 (segment (start 122.09275 92.64275) (end 122.09275 89.63025) (width 0.2) (layer "F.Cu") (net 10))
 (segment (start 122.09275 89.63025) (end 119.69375 87.23125) (width 0.2) (layer "F.Cu") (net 10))
 (segment (start 123.19375 93.74375) (end 122.09275 92.64275) (width 0.2) (layer "F.Cu") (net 10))
 (segment (start 136.443 88.1115) (end 135.38 87.0485) (width 0.2) (layer "F.Cu") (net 12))
 (segment (start 120.015 112.7804) (end 136.443 96.3524) (width 0.2) (layer "F.Cu") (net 12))
 (segment (start 120.015 126.0475) (end 120.015 112.7804) (width 0.2) (layer "F.Cu") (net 12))
 (segment (start 136.443 96.3524) (end 136.443 88.1115) (width 0.2) (layer "F.Cu") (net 12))
 (segment (start 119.0625 144.145) (end 119.0625 138.7135) (width 0.2) (layer "F.Cu") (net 2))
 (segment (start 116.68125 136.33225) (end 116.68125 97.63125) (width 0.2) (layer "F.Cu") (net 2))
 (segment (start 120.015 145.0975) (end 119.0625 144.145) (width 0.2) (layer "F.Cu") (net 2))
 (segment (start 135.38 95.60125) (end 135.38 89.5885) (width 0.2) (layer "F.Cu") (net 2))
 (segment (start 133.35 97.63125) (end 135.38 95.60125) (width 0.2) (layer "F.Cu") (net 2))
 (segment (start 116.68125 97.63125) (end 133.35 97.63125) (width 0.2) (layer "F.Cu") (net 2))
 (segment (start 119.0625 138.7135) (end 116.68125 136.33225) (width 0.2) (layer "F.Cu") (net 2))
 (segment (start 148.423 91.7855) (end 150.62 89.5885) (width 0.2) (layer "F.Cu") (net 7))
 (segment (start 139.065 126.0475) (end 148.423 116.6895) (width 0.2) (layer "F.Cu") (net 7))
 (segment (start 148.423 116.6895) (end 148.423 91.7855) (width 0.2) (layer "F.Cu") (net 7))
 (segment (start 134.324 140.3565) (end 134.324 103.3445) (width 0.2) (layer "F.Cu") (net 17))
 (segment (start 134.324 103.3445) (end 150.62 87.0485) (width 0.2) (layer "F.Cu") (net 17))
 (segment (start 139.065 145.0975) (end 134.324 140.3565) (width 0.2) (layer "F.Cu") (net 17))
 (segment (start 151.69763 84.5085) (end 150.62 84.5085) (width 0.2) (layer "F.Cu") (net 16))
 (segment (start 148.824 94.538126) (end 152.972 90.390126) (width 0.2) (layer "F.Cu") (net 16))
 (segment (start 152.972 90.390126) (end 152.972 85.78287) (width 0.2) (layer "F.Cu") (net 16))
 (segment (start 148.824 116.7565) (end 148.824 94.538126) (width 0.2) (layer "F.Cu") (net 16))
 (segment (start 158.115 126.0475) (end 148.824 116.7565) (width 0.2) (layer "F.Cu") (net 16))
 (segment (start 152.972 85.78287) (end 151.69763 84.5085) (width 0.2) (layer "F.Cu") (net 16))
 (segment (start 159.54375 115.914892) (end 167.55825 107.900392) (width 0.2) (layer "F.Cu") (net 15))
 (segment (start 158.115 145.0975) (end 159.54375 143.66875) (width 0.2) (layer "F.Cu") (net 15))
 (segment (start 157.453 72.0385) (end 149.41775 72.0385) (width 0.2) (layer "F.Cu") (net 15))
 (segment (start 149.41775 72.0385) (end 147.6375 73.81875) (width 0.2) (layer "F.Cu") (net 15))
 (segment (start 147.6375 78.986) (end 150.62 81.9685) (width 0.2) (layer "F.Cu") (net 15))
 (segment (start 147.6375 73.81875) (end 147.6375 78.986) (width 0.2) (layer "F.Cu") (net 15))
 (segment (start 167.55825 82.14375) (end 157.453 72.0385) (width 0.2) (layer "F.Cu") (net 15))
 (segment (start 167.55825 107.900392) (end 167.55825 82.14375) (width 0.2) (layer "F.Cu") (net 15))
 (segment (start 159.54375 143.66875) (end 159.54375 115.914892) (width 0.2) (layer "F.Cu") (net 15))
 (segment (start 133.35 78.9185) (end 135.38 76.8885) (width 0.2) (layer "B.Cu") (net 14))
 (segment (start 133.35 104.775) (end 133.35 107.38125) (width 0.2) (layer "B.Cu") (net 14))
 (segment (start 133.35 107.38125) (end 133.35 107.15625) (width 0.2) (layer "B.Cu") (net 14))
 (segment (start 133.35 107.38125) (end 135.625 109.65625) (width 0.2) (layer "B.Cu") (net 14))
 (segment (start 133.35 104.775) (end 133.35 78.9185) (width 0.2) (layer "B.Cu") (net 14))
 (segment (start 133.35 104.775) (end 133.35 100.0125) (width 0.2) (layer "B.Cu") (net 14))
 (segment (start 134.317 103.34825) (end 134.317 80.4915) (width 0.2) (layer "B.Cu") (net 13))
 (segment (start 135.625 104.65625) (end 134.317 103.34825) (width 0.2) (layer "B.Cu") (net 13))
 (segment (start 134.317 80.4915) (end 135.38 79.4285) (width 0.2) (layer "B.Cu") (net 13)))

